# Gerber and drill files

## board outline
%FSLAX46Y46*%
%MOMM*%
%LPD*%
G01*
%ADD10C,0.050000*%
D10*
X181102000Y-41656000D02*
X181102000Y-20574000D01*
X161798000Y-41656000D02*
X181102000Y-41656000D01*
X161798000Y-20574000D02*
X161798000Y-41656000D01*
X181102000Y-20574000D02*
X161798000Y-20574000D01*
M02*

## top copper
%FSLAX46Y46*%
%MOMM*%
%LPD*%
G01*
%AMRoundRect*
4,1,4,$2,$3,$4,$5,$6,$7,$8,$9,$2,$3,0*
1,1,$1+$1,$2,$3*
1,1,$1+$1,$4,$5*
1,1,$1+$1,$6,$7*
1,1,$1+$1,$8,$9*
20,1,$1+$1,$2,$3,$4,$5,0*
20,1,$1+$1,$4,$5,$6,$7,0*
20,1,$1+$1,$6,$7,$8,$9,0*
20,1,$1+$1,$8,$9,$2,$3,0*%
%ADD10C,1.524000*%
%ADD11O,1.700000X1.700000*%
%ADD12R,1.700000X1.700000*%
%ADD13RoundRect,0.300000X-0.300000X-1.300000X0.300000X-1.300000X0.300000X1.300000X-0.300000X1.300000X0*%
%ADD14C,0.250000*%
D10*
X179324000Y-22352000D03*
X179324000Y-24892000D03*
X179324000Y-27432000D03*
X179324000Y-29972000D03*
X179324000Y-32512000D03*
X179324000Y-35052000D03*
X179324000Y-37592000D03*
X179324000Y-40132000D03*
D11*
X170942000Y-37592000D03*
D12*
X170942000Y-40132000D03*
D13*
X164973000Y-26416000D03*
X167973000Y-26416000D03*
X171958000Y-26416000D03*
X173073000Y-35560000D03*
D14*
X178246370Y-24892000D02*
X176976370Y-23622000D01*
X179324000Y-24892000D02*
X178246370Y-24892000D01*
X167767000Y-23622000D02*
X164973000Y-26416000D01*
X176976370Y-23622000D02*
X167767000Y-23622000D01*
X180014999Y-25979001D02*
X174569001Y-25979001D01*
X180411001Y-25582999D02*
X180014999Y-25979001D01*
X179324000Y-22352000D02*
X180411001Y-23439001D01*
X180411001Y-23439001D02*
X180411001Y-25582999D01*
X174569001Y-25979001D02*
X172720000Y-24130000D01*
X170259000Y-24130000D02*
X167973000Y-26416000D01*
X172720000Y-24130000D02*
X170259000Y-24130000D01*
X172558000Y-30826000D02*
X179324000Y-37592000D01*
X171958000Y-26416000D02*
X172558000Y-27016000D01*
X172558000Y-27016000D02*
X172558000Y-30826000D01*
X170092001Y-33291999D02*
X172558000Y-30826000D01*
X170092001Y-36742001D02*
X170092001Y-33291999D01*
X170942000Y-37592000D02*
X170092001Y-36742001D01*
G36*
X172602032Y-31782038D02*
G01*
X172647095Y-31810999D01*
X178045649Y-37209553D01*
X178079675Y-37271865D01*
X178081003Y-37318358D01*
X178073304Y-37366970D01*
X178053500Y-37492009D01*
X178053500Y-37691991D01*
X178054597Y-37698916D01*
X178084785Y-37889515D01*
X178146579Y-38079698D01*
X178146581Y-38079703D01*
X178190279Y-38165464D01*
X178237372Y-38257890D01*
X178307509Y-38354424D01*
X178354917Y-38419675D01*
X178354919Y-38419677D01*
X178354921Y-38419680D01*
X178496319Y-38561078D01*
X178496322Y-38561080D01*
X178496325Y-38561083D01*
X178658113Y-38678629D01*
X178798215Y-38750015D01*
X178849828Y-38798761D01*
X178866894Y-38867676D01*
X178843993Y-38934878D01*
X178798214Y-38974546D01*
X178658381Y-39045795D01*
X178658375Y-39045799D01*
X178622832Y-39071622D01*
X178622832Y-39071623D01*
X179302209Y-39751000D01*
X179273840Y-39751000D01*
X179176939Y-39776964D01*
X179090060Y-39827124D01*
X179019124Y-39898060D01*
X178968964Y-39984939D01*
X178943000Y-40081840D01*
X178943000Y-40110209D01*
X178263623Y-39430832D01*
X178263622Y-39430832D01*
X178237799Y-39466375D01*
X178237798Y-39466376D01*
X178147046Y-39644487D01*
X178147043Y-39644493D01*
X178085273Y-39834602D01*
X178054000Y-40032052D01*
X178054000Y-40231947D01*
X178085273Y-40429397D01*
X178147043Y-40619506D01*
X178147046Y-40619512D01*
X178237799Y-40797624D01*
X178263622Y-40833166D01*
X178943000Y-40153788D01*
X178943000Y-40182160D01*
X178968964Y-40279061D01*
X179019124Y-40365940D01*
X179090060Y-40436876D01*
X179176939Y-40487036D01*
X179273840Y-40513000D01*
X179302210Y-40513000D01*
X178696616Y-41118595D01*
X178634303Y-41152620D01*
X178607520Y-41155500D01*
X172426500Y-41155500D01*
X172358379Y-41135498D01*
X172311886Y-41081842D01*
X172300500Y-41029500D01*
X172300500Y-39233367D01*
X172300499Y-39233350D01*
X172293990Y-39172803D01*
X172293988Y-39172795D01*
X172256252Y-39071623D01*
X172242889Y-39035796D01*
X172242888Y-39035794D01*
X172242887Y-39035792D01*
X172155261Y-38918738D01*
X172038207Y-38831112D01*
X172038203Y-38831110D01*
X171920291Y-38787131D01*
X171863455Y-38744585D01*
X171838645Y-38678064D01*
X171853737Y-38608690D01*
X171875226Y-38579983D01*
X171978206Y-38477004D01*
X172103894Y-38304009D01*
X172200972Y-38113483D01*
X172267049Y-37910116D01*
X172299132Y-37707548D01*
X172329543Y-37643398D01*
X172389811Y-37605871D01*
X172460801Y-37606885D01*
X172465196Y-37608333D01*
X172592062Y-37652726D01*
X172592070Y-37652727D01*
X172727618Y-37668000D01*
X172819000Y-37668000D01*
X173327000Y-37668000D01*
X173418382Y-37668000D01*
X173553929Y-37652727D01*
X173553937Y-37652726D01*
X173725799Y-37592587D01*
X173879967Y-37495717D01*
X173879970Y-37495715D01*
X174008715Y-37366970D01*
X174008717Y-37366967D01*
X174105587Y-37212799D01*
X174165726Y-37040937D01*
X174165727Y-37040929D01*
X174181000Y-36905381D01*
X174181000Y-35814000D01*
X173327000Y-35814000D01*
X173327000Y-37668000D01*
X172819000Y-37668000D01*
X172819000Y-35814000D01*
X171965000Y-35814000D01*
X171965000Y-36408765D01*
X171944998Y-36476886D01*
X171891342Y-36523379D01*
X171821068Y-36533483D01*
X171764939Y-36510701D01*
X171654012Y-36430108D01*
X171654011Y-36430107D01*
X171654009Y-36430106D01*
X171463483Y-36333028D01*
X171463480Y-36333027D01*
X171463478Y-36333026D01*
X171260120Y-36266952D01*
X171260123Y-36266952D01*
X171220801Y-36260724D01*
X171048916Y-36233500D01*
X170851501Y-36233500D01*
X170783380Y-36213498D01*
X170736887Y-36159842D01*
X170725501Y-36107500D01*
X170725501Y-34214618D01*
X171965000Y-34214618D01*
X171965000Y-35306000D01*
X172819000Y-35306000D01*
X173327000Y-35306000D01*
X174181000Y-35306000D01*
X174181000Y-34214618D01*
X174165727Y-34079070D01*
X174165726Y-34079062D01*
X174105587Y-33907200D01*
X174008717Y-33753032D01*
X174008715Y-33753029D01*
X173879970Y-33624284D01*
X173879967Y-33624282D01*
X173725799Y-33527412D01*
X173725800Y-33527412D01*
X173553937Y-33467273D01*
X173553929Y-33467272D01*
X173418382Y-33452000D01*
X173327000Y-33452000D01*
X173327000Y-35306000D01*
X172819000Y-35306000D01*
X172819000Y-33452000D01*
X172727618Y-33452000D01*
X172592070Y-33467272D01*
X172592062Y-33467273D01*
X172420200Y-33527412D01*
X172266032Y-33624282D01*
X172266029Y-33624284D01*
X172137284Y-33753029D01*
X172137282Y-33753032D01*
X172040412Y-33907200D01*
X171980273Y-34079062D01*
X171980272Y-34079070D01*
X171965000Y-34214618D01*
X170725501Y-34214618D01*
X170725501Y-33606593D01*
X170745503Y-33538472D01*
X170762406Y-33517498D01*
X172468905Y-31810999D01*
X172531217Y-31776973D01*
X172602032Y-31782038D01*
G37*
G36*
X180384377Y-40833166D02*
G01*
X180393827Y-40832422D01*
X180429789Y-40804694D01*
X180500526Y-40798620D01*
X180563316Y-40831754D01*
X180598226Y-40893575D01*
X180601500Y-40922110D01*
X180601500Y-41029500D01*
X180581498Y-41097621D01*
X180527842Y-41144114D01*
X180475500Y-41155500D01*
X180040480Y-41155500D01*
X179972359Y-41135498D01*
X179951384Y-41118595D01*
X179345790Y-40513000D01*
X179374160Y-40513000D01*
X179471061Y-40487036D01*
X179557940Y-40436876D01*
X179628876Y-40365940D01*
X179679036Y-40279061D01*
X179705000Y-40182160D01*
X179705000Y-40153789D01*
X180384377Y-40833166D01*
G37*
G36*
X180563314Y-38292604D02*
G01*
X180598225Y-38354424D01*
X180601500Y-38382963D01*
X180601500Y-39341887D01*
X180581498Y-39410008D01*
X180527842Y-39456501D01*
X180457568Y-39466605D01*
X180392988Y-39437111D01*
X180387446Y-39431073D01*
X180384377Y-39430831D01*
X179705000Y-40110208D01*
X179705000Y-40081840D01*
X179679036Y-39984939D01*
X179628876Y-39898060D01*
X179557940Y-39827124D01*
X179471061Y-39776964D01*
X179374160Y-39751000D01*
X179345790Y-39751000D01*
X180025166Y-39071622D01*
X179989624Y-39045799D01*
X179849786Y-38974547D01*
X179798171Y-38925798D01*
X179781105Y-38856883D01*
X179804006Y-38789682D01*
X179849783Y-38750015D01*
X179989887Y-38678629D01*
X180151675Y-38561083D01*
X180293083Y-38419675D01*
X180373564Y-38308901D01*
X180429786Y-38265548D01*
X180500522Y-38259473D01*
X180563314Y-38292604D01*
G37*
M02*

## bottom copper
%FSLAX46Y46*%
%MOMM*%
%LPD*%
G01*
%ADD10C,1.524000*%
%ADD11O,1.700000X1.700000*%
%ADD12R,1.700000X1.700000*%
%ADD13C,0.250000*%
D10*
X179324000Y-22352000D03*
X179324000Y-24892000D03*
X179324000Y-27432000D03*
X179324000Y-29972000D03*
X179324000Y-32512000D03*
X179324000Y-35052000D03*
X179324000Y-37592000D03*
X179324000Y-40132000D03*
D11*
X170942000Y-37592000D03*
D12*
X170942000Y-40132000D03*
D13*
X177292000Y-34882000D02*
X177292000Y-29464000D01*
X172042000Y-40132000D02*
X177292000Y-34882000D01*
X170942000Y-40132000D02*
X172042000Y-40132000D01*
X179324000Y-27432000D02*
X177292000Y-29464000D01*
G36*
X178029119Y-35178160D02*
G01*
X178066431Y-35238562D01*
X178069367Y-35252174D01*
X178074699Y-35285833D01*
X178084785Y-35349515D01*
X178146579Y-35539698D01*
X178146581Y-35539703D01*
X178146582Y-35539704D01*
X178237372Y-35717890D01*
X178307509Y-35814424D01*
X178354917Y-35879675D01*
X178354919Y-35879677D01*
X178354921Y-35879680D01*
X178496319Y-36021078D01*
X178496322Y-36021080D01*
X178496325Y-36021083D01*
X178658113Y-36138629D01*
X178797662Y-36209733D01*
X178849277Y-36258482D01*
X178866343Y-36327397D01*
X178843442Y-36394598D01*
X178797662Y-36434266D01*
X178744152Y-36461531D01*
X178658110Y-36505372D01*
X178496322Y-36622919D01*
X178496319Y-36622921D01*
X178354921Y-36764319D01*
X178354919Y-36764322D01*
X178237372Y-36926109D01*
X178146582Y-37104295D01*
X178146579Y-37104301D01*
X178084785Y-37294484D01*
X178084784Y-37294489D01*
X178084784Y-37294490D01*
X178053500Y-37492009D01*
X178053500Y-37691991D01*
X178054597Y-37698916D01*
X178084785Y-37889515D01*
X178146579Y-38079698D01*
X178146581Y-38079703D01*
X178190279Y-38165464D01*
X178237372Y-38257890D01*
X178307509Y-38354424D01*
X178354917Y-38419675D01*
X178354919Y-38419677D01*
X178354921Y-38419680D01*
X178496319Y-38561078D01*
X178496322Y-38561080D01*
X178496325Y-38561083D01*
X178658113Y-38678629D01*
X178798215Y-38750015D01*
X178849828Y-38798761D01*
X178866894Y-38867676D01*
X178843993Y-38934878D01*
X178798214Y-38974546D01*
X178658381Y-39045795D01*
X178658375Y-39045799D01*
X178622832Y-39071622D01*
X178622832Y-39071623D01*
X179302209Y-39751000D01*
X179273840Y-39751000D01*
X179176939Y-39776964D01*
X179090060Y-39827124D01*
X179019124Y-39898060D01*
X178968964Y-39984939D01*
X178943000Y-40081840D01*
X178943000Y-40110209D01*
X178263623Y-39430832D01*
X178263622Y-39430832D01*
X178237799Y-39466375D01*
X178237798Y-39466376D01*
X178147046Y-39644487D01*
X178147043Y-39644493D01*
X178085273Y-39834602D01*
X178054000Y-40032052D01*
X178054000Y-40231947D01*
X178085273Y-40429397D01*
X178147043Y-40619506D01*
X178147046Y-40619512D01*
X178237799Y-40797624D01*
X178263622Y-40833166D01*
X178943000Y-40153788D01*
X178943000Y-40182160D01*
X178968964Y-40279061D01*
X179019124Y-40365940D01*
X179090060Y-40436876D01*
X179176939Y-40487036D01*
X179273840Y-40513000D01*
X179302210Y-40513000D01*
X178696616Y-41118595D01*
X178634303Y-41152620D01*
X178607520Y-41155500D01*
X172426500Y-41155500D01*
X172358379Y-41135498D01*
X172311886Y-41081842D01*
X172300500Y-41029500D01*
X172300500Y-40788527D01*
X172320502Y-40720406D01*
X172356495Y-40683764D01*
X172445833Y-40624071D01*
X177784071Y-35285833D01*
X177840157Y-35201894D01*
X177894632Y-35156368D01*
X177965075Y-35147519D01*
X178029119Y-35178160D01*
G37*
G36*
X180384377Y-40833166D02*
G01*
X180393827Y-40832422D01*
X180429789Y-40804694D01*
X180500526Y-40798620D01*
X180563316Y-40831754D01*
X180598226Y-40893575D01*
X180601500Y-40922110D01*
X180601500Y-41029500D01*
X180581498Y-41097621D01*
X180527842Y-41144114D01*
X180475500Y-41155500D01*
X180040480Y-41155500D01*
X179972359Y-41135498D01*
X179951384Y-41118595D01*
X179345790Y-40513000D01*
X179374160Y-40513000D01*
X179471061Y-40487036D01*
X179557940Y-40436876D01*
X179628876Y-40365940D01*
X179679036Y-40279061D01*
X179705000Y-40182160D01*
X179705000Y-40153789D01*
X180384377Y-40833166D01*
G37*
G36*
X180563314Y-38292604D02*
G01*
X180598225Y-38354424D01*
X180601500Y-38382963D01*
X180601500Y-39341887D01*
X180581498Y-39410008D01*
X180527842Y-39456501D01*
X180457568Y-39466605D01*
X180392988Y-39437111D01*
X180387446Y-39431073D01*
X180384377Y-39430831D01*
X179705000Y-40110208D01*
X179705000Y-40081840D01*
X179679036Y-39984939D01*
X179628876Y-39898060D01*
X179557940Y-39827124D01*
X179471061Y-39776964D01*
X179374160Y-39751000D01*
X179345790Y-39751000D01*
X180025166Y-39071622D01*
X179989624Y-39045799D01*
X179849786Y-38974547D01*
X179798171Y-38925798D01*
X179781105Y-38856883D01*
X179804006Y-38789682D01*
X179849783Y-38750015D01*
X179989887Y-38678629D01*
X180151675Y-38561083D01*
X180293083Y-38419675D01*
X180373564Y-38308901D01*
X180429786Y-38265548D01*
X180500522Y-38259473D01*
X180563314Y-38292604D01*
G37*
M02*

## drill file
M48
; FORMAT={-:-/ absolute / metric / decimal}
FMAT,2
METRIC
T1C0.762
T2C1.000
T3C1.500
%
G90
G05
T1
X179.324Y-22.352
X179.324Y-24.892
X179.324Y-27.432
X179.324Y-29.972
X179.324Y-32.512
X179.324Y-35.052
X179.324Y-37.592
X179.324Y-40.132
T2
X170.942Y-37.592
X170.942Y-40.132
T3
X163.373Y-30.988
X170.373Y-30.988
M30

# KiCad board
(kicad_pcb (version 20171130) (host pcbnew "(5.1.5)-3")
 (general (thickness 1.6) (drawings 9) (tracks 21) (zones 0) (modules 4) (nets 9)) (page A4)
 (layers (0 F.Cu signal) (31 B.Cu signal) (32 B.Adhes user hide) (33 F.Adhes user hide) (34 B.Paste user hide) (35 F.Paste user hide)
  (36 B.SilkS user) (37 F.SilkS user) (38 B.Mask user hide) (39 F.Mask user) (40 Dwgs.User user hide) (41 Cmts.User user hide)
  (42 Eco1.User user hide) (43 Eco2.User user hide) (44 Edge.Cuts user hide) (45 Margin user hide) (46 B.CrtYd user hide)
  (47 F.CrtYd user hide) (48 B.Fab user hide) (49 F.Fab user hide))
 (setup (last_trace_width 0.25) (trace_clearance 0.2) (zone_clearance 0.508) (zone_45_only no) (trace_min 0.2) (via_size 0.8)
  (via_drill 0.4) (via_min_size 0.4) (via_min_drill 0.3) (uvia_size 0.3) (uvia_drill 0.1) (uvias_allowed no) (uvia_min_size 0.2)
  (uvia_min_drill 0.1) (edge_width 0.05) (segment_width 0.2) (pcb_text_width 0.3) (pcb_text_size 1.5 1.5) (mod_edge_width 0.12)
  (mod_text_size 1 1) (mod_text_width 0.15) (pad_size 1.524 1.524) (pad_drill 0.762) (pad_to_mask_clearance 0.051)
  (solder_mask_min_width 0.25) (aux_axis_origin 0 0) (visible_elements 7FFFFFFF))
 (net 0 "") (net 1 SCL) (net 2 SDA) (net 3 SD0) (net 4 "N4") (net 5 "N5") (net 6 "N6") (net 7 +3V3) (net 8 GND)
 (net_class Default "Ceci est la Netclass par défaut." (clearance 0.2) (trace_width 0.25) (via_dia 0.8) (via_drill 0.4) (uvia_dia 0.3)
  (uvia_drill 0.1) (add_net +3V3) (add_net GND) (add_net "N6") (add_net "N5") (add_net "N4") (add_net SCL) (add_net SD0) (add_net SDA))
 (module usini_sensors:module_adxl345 (layer F.Cu) (at 179.324 24.892 180)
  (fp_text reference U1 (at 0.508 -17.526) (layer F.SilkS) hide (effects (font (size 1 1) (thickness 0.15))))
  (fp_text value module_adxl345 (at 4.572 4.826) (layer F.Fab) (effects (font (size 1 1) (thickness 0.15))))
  (pad 8 thru_hole circle (at 0 2.54 180) (size 1.524 1.524) (drill 0.762) (layers *.Cu *.Mask) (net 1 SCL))
  (pad 7 thru_hole circle (at 0 0 180) (size 1.524 1.524) (drill 0.762) (layers *.Cu *.Mask) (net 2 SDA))
  (pad 6 thru_hole circle (at 0 -2.54 180) (size 1.524 1.524) (drill 0.762) (layers *.Cu *.Mask) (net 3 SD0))
  (pad 5 thru_hole circle (at 0 -5.08 180) (size 1.524 1.524) (drill 0.762) (layers *.Cu *.Mask) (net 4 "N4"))
  (pad 4 thru_hole circle (at 0 -7.62 180) (size 1.524 1.524) (drill 0.762) (layers *.Cu *.Mask) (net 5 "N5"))
  (pad 3 thru_hole circle (at 0 -10.16 180) (size 1.524 1.524) (drill 0.762) (layers *.Cu *.Mask) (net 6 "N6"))
  (pad 2 thru_hole circle (at 0 -12.7 180) (size 1.524 1.524) (drill 0.762) (layers *.Cu *.Mask) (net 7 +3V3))
  (pad 1 thru_hole circle (at 0 -15.24 180) (size 1.524 1.524) (drill 0.762) (layers *.Cu *.Mask) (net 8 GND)))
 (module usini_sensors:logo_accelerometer (layer B.Cu) (at 166.116 24.384 180)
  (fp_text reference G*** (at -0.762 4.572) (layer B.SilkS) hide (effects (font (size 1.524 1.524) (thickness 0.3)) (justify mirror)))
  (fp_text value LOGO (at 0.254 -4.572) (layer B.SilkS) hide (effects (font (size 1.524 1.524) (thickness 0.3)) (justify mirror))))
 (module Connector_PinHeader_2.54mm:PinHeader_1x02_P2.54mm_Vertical (layer F.Cu) (at 170.942 40.132 180)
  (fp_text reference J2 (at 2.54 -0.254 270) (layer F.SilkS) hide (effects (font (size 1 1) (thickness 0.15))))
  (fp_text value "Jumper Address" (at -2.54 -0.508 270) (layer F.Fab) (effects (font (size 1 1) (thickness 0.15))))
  (pad 2 thru_hole oval (at 0 2.54 180) (size 1.7 1.7) (drill 1) (layers *.Cu *.Mask) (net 7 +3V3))
  (pad 1 thru_hole rect (at 0 0 180) (size 1.7 1.7) (drill 1) (layers *.Cu *.Mask) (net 3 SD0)))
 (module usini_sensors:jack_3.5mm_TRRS (layer F.Cu) (at 168.148 30.988)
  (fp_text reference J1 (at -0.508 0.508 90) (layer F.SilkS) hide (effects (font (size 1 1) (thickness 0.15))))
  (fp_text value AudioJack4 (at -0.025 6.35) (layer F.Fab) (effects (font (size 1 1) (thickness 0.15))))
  (pad "" np_thru_hole circle (at 2.225 0) (size 1.5 1.5) (drill 1.5) (layers *.Cu *.Mask))
  (pad "" np_thru_hole circle (at -4.775 0) (size 1.5 1.5) (drill 1.5) (layers *.Cu *.Mask))
  (pad R2 smd roundrect (at -3.175 -4.572) (size 1.2 3.2) (layers F.Cu F.Paste F.Mask) (roundrect_rratio 0.25) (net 2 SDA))
  (pad R1 smd roundrect (at -0.175 -4.572) (size 1.2 3.2) (layers F.Cu F.Paste F.Mask) (roundrect_rratio 0.25) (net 1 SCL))
  (pad T smd roundrect (at 3.81 -4.572) (size 1.2 3.2) (layers F.Cu F.Paste F.Mask) (roundrect_rratio 0.25) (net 7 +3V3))
  (pad S smd roundrect (at 4.925 4.572) (size 1.2 3.2) (layers F.Cu F.Paste F.Mask) (roundrect_rratio 0.25) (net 8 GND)))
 (gr_line (start 181.102 41.656) (end 181.102 20.574) (layer Edge.Cuts) (width 0.05))
 (gr_line (start 161.798 41.656) (end 181.102 41.656) (layer Edge.Cuts) (width 0.05))
 (gr_line (start 161.798 20.574) (end 161.798 41.656) (layer Edge.Cuts) (width 0.05))
 (gr_line (start 181.102 20.574) (end 161.798 20.574) (layer Edge.Cuts) (width 0.05))
 (segment (start 178.24637 24.892) (end 176.97637 23.622) (width 0.25) (layer F.Cu) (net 2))
 (segment (start 179.324 24.892) (end 178.24637 24.892) (width 0.25) (layer F.Cu) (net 2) (status 10))
 (segment (start 167.767 23.622) (end 164.973 26.416) (width 0.25) (layer F.Cu) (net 2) (status 20))
 (segment (start 176.97637 23.622) (end 167.767 23.622) (width 0.25) (layer F.Cu) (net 2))
 (segment (start 180.014999 25.979001) (end 174.569001 25.979001) (width 0.25) (layer F.Cu) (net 1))
 (segment (start 180.411001 25.582999) (end 180.014999 25.979001) (width 0.25) (layer F.Cu) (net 1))
 (segment (start 179.324 22.352) (end 180.411001 23.439001) (width 0.25) (layer F.Cu) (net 1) (status 10))
 (segment (start 180.411001 23.439001) (end 180.411001 25.582999) (width 0.25) (layer F.Cu) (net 1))
 (segment (start 174.569001 25.979001) (end 172.72 24.13) (width 0.25) (layer F.Cu) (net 1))
 (segment (start 170.259 24.13) (end 167.973 26.416) (width 0.25) (layer F.Cu) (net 1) (status 20))
 (segment (start 172.72 24.13) (end 170.259 24.13) (width 0.25) (layer F.Cu) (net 1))
 (segment (start 172.558 30.826) (end 179.324 37.592) (width 0.25) (layer F.Cu) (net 7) (status 20))
 (segment (start 171.958 26.416) (end 172.558 27.016) (width 0.25) (layer F.Cu) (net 7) (status 10))
 (segment (start 172.558 27.016) (end 172.558 30.826) (width 0.25) (layer F.Cu) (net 7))
 (segment (start 170.092001 33.291999) (end 172.558 30.826) (width 0.25) (layer F.Cu) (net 7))
 (segment (start 170.092001 36.742001) (end 170.092001 33.291999) (width 0.25) (layer F.Cu) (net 7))
 (segment (start 170.942 37.592) (end 170.092001 36.742001) (width 0.25) (layer F.Cu) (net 7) (status 10))
 (segment (start 177.292 34.882) (end 177.292 29.464) (width 0.25) (layer B.Cu) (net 3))
 (segment (start 172.042 40.132) (end 177.292 34.882) (width 0.25) (layer B.Cu) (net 3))
 (segment (start 170.942 40.132) (end 172.042 40.132) (width 0.25) (layer B.Cu) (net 3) (status 10))
 (segment (start 179.324 27.432) (end 177.292 29.464) (width 0.25) (layer B.Cu) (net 3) (status 10))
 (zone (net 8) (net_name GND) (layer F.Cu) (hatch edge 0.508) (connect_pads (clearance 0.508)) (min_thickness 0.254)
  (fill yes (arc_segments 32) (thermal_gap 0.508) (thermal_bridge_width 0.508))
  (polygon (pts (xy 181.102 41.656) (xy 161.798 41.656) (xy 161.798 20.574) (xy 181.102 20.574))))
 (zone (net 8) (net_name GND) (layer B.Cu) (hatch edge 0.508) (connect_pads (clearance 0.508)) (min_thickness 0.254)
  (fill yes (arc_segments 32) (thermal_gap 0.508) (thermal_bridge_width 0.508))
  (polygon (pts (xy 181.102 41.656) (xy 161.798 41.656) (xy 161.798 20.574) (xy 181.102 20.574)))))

